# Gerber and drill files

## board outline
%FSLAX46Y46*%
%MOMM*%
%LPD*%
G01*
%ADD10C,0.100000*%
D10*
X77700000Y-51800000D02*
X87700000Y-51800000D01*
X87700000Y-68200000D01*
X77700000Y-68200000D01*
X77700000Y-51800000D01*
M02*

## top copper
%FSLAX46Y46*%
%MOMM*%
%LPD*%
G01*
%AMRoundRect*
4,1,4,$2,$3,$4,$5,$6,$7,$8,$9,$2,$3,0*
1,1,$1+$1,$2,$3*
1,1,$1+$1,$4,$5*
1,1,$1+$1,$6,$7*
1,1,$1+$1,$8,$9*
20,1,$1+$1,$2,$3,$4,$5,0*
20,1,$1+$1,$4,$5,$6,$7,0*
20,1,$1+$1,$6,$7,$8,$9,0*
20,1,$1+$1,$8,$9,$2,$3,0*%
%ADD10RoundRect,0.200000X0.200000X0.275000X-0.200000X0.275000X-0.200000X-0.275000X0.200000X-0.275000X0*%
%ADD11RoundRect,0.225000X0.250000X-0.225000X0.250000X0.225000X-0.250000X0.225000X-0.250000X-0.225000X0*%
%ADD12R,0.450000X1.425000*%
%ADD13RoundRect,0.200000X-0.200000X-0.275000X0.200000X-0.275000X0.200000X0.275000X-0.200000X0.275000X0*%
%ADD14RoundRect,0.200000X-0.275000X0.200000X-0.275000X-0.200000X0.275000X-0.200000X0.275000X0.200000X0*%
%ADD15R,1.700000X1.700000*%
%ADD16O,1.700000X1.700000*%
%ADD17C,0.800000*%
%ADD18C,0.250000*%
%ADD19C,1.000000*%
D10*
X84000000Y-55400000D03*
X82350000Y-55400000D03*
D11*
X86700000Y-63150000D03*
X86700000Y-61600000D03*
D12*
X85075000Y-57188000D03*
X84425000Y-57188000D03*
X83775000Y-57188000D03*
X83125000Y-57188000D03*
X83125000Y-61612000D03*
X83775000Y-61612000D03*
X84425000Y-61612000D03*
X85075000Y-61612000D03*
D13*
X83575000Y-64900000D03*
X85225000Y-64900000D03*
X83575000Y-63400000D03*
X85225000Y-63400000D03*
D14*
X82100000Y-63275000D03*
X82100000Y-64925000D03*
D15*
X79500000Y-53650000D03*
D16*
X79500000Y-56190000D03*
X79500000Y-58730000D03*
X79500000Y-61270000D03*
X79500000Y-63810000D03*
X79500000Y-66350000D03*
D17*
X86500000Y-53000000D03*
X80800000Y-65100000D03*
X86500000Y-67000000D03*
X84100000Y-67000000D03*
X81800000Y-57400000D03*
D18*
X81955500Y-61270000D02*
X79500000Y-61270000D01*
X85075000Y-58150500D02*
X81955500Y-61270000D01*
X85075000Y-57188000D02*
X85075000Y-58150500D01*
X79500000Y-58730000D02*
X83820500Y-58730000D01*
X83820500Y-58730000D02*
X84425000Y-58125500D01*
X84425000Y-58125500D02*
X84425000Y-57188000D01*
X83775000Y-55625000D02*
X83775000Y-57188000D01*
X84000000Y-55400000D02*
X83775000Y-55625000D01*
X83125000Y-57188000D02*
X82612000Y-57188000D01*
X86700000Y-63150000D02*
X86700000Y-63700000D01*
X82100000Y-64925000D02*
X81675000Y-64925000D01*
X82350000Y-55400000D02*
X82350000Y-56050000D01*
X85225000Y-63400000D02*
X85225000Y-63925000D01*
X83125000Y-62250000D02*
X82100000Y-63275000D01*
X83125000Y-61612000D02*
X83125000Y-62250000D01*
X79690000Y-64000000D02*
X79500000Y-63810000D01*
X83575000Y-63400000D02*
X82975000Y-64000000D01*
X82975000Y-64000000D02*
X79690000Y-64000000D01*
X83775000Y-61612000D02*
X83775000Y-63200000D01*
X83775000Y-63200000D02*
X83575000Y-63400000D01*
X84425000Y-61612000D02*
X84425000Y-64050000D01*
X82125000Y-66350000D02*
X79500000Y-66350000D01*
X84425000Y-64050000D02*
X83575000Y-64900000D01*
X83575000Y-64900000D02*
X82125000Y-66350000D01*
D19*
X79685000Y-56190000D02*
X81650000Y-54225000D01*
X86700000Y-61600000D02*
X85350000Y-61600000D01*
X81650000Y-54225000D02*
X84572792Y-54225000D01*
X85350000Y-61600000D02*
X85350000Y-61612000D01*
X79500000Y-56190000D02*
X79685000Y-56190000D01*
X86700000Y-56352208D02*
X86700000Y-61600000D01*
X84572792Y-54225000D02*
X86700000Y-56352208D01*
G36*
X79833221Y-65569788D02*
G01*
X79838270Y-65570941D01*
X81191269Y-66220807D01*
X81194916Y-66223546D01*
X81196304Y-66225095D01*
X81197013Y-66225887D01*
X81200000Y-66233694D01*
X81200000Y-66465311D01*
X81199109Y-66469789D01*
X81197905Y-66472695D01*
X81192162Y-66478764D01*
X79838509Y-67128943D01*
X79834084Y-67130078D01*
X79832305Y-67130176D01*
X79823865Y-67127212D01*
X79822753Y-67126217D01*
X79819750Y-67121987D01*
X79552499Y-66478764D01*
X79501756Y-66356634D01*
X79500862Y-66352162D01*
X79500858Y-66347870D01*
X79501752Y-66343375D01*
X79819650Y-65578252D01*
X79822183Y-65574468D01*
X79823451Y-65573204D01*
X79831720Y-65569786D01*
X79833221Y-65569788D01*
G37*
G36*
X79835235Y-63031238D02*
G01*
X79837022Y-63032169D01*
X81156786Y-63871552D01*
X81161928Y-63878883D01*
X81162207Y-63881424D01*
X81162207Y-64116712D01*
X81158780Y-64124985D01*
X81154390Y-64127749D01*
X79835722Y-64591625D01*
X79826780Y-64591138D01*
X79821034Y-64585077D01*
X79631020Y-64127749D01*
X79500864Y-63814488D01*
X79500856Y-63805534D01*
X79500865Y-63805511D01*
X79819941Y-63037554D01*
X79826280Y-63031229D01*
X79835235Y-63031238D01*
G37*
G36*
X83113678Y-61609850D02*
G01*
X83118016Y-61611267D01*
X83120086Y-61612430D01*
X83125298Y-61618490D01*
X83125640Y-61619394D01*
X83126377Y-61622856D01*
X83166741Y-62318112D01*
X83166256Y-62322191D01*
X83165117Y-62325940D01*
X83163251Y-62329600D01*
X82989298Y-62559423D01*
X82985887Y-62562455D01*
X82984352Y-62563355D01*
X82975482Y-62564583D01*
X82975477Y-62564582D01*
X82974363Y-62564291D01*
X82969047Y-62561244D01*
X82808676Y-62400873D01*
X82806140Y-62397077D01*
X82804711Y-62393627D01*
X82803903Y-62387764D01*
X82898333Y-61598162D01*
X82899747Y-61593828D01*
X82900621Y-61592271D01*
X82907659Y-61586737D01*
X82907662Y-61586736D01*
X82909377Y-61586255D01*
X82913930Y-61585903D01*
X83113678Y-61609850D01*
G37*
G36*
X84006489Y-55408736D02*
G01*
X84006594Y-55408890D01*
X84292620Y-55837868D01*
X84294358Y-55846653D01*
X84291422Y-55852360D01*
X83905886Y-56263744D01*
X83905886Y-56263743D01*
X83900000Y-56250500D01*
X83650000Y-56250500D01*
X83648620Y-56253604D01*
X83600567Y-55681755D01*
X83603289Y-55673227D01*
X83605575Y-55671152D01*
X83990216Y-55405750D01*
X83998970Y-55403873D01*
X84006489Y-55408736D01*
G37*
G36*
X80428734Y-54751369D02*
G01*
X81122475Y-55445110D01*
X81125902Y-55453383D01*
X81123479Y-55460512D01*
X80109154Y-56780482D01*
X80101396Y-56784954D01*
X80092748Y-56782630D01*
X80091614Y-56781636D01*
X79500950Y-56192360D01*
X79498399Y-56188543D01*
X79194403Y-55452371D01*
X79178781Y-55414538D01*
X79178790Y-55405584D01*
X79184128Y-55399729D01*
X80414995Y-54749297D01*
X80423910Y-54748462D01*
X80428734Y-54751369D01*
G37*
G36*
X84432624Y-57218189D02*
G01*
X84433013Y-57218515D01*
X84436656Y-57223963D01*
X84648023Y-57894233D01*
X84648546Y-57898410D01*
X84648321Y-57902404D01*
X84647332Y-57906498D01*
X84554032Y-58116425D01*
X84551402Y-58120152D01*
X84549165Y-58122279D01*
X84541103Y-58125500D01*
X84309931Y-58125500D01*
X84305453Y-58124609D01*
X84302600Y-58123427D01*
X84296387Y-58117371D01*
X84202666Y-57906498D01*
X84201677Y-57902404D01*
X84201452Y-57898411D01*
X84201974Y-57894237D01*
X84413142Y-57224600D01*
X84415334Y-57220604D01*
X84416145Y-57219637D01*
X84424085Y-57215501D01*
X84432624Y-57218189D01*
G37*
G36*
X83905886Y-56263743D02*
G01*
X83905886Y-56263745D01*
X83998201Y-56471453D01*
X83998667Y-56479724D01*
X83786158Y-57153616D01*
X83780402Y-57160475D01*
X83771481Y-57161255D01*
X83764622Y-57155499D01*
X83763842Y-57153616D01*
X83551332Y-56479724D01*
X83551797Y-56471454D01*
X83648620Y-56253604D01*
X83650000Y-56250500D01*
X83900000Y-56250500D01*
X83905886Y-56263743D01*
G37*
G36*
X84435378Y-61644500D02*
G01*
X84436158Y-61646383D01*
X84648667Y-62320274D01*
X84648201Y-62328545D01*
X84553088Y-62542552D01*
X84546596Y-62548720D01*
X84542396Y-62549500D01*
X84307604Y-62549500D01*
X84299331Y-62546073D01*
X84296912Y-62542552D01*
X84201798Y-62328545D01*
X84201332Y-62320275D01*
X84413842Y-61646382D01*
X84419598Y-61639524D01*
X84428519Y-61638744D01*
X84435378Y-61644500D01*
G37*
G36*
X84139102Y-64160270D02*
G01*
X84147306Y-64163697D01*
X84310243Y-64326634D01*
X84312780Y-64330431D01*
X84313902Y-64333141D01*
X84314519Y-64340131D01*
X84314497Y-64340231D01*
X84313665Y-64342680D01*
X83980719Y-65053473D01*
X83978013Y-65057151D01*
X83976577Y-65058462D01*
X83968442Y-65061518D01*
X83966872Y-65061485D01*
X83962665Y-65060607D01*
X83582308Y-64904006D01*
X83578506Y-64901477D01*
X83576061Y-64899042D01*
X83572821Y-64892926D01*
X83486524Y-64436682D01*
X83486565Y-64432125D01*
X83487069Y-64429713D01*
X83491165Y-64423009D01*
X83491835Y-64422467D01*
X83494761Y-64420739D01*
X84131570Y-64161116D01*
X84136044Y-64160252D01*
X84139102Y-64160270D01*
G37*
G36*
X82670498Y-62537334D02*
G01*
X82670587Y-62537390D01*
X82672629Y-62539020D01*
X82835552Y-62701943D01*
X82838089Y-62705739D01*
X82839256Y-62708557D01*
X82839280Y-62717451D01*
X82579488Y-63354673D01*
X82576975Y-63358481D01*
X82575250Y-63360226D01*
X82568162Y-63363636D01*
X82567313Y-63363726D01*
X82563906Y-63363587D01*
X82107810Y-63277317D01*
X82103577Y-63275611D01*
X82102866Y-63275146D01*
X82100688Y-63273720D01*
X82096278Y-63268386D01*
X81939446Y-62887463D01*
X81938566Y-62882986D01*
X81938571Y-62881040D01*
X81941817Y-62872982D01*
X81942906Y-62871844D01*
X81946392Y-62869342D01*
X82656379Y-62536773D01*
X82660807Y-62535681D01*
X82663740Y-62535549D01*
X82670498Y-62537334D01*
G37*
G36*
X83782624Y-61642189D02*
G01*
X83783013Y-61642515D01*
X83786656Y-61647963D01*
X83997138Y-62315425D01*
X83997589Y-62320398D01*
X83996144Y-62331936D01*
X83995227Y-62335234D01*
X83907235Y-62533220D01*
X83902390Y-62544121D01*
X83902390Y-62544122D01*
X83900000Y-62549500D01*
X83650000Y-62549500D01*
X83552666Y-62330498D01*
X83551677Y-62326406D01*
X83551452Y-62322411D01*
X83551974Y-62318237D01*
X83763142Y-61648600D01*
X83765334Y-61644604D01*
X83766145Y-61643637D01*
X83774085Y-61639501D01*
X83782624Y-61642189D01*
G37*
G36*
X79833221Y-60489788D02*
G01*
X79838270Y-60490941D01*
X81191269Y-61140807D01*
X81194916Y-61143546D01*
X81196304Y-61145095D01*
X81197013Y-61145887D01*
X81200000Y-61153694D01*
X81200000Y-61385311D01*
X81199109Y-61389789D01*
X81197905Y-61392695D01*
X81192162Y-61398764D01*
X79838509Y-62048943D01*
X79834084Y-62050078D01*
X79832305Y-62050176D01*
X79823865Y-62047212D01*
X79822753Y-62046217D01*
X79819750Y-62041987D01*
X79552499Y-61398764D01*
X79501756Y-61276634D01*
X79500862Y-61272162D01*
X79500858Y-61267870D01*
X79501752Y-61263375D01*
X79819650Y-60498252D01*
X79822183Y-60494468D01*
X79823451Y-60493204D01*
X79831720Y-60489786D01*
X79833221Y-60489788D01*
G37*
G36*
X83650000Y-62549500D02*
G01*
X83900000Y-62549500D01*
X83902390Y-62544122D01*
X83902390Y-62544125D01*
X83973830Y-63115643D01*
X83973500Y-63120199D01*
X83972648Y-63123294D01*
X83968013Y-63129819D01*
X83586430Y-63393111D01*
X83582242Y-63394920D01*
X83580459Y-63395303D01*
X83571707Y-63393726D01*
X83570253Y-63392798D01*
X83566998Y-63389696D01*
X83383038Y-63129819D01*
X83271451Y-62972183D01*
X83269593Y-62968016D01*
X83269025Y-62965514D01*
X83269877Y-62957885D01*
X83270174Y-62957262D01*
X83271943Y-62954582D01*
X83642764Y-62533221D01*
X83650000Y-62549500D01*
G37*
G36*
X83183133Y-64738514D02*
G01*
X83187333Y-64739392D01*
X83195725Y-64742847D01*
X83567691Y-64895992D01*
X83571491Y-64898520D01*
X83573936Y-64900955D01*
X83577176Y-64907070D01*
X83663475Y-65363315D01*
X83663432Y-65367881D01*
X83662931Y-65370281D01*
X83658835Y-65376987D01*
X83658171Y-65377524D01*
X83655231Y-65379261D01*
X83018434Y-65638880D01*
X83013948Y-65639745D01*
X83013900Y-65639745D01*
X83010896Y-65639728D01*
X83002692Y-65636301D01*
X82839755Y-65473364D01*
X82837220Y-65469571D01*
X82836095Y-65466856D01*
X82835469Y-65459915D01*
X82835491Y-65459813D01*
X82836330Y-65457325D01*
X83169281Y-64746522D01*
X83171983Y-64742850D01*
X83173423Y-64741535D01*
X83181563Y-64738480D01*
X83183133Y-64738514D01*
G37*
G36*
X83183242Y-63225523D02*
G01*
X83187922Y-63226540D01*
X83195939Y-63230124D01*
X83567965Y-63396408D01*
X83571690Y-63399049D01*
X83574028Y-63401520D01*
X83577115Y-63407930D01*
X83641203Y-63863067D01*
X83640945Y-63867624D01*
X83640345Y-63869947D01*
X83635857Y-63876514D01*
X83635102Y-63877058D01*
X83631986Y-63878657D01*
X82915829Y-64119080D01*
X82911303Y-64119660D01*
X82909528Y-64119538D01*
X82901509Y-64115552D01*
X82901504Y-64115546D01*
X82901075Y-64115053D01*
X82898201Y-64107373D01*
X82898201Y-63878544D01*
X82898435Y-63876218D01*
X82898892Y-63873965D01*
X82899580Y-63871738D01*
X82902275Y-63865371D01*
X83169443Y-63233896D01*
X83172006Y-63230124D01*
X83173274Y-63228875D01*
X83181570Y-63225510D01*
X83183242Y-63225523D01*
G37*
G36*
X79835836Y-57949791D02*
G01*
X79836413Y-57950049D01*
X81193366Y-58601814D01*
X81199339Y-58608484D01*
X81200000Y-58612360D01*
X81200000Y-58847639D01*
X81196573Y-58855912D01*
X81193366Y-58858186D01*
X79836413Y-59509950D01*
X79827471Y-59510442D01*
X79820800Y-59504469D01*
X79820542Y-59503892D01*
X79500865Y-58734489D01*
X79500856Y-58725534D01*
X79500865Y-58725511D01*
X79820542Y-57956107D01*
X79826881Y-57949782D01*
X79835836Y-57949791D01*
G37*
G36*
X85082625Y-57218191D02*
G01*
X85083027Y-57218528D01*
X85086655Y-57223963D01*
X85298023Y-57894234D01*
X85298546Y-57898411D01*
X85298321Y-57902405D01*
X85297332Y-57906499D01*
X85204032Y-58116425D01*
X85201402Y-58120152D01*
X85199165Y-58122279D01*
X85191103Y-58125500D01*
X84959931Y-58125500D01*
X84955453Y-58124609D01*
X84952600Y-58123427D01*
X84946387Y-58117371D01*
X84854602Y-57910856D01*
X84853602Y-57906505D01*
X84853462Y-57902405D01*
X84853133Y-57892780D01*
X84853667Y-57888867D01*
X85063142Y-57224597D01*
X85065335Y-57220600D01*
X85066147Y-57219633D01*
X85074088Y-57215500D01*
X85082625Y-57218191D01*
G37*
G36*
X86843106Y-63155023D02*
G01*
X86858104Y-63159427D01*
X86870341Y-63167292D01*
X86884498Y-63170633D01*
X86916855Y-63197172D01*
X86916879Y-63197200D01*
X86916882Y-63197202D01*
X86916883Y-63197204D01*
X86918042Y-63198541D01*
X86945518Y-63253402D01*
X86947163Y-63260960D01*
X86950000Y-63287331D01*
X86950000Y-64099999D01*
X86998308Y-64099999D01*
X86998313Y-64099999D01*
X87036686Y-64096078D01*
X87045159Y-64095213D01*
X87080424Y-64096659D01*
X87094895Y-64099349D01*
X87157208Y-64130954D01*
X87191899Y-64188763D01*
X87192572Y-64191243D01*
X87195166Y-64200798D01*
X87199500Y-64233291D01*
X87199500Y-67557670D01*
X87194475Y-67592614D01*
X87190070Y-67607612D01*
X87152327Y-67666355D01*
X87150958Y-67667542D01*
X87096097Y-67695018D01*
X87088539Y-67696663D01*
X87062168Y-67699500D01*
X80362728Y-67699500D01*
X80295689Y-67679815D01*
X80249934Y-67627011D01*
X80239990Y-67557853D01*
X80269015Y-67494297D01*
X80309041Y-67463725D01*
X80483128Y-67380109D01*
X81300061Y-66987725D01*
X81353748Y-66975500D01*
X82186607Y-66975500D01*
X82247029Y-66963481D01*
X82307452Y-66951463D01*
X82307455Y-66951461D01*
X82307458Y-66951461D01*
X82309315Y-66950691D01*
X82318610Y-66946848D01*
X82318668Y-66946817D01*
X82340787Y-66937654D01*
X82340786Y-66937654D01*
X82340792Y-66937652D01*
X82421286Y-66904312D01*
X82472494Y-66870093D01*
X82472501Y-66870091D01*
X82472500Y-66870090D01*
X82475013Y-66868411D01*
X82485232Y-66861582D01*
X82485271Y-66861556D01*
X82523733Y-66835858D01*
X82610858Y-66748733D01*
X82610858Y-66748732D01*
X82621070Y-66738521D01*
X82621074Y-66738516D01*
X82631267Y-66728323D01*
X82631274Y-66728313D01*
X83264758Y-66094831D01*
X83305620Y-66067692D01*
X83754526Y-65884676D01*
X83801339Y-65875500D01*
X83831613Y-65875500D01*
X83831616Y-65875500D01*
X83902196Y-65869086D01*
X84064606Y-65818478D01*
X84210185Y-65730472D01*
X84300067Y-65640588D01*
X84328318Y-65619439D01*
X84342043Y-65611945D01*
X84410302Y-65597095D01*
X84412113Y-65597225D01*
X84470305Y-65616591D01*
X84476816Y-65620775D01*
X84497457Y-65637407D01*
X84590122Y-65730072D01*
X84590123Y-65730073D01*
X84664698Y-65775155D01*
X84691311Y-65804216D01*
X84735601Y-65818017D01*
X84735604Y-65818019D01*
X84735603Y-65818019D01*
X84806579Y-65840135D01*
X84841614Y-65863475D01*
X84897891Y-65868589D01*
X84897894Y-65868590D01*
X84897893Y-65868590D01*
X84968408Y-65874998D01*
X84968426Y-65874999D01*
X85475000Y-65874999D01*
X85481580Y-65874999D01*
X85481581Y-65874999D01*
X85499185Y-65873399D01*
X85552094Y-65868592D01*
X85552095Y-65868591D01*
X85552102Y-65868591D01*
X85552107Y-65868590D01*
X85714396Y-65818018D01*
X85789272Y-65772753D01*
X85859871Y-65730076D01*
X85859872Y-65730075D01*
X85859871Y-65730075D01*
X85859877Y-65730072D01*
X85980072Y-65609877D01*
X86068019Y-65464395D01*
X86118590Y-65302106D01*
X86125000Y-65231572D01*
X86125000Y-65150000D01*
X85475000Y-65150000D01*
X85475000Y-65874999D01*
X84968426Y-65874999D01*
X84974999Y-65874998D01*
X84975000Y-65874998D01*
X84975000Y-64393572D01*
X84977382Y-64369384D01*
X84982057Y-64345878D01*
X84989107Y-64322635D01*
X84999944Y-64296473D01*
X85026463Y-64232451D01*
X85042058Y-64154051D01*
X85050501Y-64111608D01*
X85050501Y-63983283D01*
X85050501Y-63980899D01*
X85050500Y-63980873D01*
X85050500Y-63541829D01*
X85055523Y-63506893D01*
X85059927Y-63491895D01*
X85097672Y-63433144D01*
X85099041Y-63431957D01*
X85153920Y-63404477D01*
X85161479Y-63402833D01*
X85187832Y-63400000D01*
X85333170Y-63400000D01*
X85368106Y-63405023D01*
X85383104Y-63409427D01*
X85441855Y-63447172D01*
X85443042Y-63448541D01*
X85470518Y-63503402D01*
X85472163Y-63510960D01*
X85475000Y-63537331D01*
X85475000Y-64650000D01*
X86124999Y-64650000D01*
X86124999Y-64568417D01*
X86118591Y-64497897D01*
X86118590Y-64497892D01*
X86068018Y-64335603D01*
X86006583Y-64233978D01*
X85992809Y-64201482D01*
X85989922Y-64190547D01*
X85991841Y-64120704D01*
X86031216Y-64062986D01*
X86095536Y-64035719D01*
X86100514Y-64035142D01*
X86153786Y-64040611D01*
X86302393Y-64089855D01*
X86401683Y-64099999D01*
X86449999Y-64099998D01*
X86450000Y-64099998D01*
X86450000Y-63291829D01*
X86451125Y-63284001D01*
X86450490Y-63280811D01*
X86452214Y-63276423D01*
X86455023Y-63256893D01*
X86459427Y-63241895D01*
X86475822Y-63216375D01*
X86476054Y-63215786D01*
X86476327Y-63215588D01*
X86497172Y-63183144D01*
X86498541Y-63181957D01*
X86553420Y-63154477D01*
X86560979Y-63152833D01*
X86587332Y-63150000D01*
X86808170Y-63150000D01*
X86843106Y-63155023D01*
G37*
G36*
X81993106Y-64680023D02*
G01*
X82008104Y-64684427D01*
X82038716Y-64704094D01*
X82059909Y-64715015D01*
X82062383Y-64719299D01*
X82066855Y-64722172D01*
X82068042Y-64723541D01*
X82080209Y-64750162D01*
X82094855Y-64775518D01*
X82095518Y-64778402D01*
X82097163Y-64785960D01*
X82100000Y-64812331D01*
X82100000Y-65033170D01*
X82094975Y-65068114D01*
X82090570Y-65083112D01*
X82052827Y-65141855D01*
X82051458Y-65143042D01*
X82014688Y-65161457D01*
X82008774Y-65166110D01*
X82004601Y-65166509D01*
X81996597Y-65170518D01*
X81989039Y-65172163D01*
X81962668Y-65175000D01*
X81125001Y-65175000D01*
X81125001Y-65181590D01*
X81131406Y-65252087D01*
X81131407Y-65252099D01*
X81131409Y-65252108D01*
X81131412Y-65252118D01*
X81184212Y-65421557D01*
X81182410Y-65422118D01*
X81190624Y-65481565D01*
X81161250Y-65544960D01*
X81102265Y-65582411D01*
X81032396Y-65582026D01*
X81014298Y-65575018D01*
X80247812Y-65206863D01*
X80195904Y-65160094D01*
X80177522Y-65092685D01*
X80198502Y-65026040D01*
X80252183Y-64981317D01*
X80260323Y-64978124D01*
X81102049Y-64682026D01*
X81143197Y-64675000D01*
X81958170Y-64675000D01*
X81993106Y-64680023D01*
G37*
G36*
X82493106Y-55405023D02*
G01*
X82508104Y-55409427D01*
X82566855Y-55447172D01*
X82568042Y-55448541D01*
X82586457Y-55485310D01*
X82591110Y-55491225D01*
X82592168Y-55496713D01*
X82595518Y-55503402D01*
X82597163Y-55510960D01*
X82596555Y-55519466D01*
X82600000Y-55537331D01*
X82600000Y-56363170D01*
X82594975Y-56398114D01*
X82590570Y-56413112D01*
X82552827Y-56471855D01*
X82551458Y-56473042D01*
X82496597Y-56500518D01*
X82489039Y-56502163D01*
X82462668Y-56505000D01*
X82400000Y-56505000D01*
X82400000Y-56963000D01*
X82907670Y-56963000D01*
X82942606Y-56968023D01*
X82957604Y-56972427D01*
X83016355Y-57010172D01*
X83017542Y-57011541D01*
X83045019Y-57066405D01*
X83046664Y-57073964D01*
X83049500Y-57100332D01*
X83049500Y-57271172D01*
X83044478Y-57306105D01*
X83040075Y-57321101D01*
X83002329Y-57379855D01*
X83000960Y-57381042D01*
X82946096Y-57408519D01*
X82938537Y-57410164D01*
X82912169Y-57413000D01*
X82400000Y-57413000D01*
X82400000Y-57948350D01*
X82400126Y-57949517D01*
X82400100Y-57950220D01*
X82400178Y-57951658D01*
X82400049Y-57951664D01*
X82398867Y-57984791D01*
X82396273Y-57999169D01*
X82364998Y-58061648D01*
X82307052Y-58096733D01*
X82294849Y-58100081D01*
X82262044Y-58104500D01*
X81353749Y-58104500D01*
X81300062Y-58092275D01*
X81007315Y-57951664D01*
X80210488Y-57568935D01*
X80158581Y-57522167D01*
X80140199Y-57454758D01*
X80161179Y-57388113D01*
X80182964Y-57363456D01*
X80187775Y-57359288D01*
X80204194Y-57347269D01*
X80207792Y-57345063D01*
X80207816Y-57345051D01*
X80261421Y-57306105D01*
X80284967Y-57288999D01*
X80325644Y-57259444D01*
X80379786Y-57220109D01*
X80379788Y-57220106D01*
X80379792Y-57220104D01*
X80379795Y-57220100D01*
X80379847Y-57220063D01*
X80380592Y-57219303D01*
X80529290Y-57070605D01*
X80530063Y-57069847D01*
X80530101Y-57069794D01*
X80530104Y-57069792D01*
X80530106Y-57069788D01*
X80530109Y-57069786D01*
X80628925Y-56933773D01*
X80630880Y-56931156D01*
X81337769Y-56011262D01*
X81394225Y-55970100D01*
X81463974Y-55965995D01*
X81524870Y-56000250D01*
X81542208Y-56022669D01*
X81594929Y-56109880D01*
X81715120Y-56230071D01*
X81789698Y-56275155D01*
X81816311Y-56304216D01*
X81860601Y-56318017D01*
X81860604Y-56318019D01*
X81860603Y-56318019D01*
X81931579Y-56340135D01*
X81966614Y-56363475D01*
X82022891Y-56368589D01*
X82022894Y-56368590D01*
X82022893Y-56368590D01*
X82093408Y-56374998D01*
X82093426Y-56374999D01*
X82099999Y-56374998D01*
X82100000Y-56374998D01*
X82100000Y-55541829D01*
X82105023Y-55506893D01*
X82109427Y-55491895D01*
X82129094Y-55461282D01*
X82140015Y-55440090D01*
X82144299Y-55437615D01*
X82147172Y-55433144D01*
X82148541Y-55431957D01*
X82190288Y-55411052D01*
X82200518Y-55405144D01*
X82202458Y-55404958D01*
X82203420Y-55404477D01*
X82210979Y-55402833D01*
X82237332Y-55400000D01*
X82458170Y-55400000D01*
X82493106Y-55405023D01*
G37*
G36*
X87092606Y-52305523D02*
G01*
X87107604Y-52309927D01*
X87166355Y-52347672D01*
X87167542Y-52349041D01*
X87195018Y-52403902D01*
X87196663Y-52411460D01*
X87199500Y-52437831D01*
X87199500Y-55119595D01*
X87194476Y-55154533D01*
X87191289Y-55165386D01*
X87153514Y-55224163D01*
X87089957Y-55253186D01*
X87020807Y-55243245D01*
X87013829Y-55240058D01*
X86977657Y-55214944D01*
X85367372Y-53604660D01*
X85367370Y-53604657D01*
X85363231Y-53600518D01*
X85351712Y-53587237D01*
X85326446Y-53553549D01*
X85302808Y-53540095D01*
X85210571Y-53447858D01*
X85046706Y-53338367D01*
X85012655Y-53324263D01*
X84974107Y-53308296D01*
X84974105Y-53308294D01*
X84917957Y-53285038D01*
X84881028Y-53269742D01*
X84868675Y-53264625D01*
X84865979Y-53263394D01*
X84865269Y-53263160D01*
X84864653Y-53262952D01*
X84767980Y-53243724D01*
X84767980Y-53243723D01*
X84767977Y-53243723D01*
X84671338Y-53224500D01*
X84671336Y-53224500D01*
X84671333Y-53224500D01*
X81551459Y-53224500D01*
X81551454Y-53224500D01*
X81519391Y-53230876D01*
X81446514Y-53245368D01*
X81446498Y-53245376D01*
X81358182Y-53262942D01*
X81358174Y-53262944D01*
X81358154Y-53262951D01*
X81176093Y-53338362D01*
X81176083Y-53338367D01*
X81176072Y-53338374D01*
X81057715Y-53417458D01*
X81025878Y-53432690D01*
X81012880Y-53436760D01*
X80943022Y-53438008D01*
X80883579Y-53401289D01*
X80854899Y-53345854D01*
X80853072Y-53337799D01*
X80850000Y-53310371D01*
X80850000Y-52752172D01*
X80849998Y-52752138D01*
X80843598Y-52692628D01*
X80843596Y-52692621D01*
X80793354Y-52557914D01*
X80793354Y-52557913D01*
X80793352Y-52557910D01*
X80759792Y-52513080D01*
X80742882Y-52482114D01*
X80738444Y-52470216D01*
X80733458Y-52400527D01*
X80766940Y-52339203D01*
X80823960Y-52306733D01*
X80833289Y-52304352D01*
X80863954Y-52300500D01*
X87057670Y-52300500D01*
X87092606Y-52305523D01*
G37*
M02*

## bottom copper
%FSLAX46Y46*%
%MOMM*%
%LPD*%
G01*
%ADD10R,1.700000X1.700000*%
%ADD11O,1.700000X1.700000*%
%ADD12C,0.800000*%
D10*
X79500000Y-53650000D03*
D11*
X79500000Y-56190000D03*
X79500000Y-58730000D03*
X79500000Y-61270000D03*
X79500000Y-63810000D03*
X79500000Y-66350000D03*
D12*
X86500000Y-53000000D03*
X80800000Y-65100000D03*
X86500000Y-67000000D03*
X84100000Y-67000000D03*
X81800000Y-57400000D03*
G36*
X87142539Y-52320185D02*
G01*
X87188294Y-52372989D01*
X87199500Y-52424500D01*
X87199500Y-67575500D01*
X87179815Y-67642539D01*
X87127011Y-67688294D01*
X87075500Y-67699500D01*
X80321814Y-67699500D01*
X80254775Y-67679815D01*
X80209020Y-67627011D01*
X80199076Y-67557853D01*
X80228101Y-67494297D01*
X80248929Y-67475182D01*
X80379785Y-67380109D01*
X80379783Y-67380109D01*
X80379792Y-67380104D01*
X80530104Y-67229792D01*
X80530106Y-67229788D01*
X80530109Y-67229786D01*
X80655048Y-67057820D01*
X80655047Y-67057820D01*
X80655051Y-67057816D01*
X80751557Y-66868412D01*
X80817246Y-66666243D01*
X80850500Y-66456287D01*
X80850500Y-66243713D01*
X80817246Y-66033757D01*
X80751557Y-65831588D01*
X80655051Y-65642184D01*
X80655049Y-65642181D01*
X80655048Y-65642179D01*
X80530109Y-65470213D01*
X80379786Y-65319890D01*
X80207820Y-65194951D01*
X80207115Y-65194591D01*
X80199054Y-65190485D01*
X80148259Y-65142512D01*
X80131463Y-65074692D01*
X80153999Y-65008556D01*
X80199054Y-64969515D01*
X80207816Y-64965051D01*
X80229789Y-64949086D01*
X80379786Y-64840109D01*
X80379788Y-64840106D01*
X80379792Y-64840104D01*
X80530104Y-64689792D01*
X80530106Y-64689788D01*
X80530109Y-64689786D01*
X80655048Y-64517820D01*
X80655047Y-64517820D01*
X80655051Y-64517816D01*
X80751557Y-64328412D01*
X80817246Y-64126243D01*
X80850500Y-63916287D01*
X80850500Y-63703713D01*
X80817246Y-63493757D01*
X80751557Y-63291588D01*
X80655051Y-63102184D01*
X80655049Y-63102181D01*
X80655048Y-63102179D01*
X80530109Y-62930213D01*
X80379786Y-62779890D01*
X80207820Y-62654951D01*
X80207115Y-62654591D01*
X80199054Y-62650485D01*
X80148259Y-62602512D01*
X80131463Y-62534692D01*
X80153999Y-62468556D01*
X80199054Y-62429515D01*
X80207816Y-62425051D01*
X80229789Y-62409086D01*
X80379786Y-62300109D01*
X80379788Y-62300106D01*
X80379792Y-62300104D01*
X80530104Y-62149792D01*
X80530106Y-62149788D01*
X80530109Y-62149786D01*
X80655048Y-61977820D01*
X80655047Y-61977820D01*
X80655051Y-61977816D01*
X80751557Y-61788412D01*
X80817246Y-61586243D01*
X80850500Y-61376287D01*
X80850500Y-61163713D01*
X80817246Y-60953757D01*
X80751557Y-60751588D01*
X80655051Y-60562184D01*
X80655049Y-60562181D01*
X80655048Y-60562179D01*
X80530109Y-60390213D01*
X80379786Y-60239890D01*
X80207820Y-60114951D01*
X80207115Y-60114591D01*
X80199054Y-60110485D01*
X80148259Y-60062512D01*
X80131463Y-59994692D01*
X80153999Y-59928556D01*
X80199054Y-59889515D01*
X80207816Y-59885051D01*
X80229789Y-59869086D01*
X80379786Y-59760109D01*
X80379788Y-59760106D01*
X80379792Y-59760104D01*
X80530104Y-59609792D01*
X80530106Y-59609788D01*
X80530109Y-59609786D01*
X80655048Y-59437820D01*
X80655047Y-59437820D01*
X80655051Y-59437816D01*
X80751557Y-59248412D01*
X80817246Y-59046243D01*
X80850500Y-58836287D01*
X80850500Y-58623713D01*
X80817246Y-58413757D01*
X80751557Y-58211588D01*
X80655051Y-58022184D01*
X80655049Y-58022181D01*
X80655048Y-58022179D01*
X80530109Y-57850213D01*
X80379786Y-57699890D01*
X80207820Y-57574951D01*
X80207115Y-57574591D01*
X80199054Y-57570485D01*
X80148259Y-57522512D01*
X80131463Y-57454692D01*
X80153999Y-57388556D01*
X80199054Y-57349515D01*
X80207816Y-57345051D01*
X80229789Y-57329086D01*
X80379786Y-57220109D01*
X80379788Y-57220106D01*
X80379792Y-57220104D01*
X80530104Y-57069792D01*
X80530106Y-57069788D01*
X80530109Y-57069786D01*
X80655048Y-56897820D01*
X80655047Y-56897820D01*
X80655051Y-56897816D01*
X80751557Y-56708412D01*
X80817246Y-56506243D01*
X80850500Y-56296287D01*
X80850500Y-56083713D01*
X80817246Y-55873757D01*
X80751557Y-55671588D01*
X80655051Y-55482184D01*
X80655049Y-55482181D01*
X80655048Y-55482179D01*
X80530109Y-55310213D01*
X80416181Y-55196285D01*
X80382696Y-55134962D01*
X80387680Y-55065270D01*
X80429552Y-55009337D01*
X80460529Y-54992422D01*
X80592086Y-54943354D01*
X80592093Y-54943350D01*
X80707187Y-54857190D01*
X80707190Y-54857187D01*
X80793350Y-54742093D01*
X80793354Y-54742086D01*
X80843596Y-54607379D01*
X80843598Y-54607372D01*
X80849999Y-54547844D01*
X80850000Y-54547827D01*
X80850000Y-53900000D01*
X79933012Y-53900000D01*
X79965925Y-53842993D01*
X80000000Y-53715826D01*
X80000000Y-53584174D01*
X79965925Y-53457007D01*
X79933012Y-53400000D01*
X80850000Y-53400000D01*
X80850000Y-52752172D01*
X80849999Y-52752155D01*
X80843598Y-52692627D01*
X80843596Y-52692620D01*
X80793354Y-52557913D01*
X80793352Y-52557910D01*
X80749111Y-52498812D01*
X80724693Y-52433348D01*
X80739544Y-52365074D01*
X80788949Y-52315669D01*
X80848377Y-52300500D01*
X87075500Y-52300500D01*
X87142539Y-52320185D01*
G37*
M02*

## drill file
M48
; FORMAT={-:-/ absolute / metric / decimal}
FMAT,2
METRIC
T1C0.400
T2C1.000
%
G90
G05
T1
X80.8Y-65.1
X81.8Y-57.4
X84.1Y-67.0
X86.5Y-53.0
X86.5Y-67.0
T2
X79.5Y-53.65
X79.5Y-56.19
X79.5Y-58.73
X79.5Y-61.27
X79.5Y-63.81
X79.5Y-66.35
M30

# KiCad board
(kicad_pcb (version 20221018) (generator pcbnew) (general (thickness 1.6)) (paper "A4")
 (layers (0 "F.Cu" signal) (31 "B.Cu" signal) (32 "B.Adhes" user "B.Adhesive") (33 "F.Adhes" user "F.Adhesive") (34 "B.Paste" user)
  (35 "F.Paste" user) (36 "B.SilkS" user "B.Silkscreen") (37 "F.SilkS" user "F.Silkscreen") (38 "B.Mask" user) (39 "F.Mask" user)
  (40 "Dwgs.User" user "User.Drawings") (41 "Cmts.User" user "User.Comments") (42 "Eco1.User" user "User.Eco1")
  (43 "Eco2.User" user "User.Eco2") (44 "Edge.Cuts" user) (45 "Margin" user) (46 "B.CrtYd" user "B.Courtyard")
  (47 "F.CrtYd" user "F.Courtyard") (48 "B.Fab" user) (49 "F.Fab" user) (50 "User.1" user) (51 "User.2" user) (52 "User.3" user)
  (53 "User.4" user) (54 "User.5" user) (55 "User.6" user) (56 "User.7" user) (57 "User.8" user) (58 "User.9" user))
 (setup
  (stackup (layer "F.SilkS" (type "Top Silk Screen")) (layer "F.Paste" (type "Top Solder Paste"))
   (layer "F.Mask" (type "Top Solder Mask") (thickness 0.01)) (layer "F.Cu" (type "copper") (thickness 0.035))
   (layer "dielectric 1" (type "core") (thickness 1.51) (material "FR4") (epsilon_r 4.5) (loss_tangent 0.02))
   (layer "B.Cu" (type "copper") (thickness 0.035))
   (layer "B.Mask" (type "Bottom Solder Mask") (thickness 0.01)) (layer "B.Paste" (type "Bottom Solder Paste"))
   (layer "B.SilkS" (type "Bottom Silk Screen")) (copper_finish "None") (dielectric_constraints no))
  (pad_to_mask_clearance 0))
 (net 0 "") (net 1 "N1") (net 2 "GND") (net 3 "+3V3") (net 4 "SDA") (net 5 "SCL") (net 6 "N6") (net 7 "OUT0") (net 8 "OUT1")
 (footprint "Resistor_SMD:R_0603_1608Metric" (layer "F.Cu") (at 83.175 55.4 180)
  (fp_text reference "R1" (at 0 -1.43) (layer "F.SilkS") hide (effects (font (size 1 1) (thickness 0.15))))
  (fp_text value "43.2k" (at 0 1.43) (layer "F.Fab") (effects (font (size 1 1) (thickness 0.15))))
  (pad "1" smd roundrect (at -0.825 0 180) (size 0.8 0.95) (layers "F.Cu" "F.Paste" "F.Mask") (roundrect_rratio 0.25) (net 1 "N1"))
  (pad "2" smd roundrect (at 0.825 0 180) (size 0.8 0.95) (layers "F.Cu" "F.Paste" "F.Mask") (roundrect_rratio 0.25) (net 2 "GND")))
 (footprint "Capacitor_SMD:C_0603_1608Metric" (layer "F.Cu") (at 86.7 62.375 90)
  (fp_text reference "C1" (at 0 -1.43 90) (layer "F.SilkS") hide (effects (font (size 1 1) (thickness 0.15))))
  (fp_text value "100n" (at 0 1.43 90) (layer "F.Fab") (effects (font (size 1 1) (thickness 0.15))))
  (pad "1" smd roundrect (at -0.775 0 90) (size 0.9 0.95) (layers "F.Cu" "F.Paste" "F.Mask") (roundrect_rratio 0.25) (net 2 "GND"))
  (pad "2" smd roundrect (at 0.775 0 90) (size 0.9 0.95) (layers "F.Cu" "F.Paste" "F.Mask") (roundrect_rratio 0.25) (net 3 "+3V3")))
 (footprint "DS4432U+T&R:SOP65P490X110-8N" (layer "F.Cu") (at 84.1 59.4 -90)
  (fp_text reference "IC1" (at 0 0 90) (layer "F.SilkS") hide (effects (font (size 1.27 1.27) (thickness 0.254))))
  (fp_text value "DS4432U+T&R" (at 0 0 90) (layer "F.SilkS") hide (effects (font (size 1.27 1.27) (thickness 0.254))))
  (pad "1" smd rect (at -2.212 -0.975) (size 0.45 1.425) (layers "F.Cu" "F.Paste" "F.Mask") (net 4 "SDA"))
  (pad "2" smd rect (at -2.212 -0.325) (size 0.45 1.425) (layers "F.Cu" "F.Paste" "F.Mask") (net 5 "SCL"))
  (pad "3" smd rect (at -2.212 0.325) (size 0.45 1.425) (layers "F.Cu" "F.Paste" "F.Mask") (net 1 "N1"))
  (pad "4" smd rect (at -2.212 0.975) (size 0.45 1.425) (layers "F.Cu" "F.Paste" "F.Mask") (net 2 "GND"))
  (pad "5" smd rect (at 2.212 0.975) (size 0.45 1.425) (layers "F.Cu" "F.Paste" "F.Mask") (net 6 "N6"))
  (pad "6" smd rect (at 2.212 0.325) (size 0.45 1.425) (layers "F.Cu" "F.Paste" "F.Mask") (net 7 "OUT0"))
  (pad "7" smd rect (at 2.212 -0.325) (size 0.45 1.425) (layers "F.Cu" "F.Paste" "F.Mask") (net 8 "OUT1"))
  (pad "8" smd rect (at 2.212 -0.975) (size 0.45 1.425) (layers "F.Cu" "F.Paste" "F.Mask") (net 3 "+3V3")))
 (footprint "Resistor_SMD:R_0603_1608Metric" (layer "F.Cu") (at 84.4 64.9)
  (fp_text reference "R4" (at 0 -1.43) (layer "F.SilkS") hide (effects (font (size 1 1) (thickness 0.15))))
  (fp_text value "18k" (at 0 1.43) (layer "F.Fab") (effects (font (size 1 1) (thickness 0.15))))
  (pad "1" smd roundrect (at -0.825 0) (size 0.8 0.95) (layers "F.Cu" "F.Paste" "F.Mask") (roundrect_rratio 0.25) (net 8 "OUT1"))
  (pad "2" smd roundrect (at 0.825 0) (size 0.8 0.95) (layers "F.Cu" "F.Paste" "F.Mask") (roundrect_rratio 0.25) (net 2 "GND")))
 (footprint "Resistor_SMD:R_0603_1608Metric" (layer "F.Cu") (at 84.4 63.4)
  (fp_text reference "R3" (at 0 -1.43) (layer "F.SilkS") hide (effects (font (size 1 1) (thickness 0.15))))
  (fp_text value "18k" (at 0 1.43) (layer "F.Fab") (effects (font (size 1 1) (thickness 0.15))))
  (pad "1" smd roundrect (at -0.825 0) (size 0.8 0.95) (layers "F.Cu" "F.Paste" "F.Mask") (roundrect_rratio 0.25) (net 7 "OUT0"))
  (pad "2" smd roundrect (at 0.825 0) (size 0.8 0.95) (layers "F.Cu" "F.Paste" "F.Mask") (roundrect_rratio 0.25) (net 2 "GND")))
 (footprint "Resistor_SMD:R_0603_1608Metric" (layer "F.Cu") (at 82.1 64.1 -90)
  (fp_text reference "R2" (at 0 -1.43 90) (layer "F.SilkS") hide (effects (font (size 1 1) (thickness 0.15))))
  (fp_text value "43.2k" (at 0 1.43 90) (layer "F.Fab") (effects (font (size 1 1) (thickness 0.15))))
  (pad "1" smd roundrect (at -0.825 0 270) (size 0.8 0.95) (layers "F.Cu" "F.Paste" "F.Mask") (roundrect_rratio 0.25) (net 6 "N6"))
  (pad "2" smd roundrect (at 0.825 0 270) (size 0.8 0.95) (layers "F.Cu" "F.Paste" "F.Mask") (roundrect_rratio 0.25) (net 2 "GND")))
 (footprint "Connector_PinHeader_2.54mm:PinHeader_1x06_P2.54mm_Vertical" (layer "B.Cu") (at 79.5 53.65 180)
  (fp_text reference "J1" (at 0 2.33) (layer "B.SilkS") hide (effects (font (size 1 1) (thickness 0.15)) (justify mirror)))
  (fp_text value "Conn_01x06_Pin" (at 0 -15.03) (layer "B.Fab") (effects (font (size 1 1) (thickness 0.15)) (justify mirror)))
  (pad "1" thru_hole rect (at 0 0 180) (size 1.7 1.7) (drill 1) (layers "*.Cu" "*.Mask") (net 2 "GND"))
  (pad "2" thru_hole oval (at 0 -2.54 180) (size 1.7 1.7) (drill 1) (layers "*.Cu" "*.Mask") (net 3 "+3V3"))
  (pad "3" thru_hole oval (at 0 -5.08 180) (size 1.7 1.7) (drill 1) (layers "*.Cu" "*.Mask") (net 5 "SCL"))
  (pad "4" thru_hole oval (at 0 -7.62 180) (size 1.7 1.7) (drill 1) (layers "*.Cu" "*.Mask") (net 4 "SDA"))
  (pad "5" thru_hole oval (at 0 -10.16 180) (size 1.7 1.7) (drill 1) (layers "*.Cu" "*.Mask") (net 7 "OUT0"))
  (pad "6" thru_hole oval (at 0 -12.7 180) (size 1.7 1.7) (drill 1) (layers "*.Cu" "*.Mask") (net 8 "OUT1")))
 (gr_rect (start 77.7 51.8) (end 87.7 68.2) (stroke (width 0.1) (type default)) (fill none) (layer "Edge.Cuts"))
 (segment (start 81.9555 61.27) (end 79.5 61.27) (width 0.25) (layer "F.Cu") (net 4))
 (segment (start 85.075 58.1505) (end 81.9555 61.27) (width 0.25) (layer "F.Cu") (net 4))
 (segment (start 85.075 57.188) (end 85.075 58.1505) (width 0.25) (layer "F.Cu") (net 4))
 (segment (start 79.5 58.73) (end 83.8205 58.73) (width 0.25) (layer "F.Cu") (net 5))
 (segment (start 83.8205 58.73) (end 84.425 58.1255) (width 0.25) (layer "F.Cu") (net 5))
 (segment (start 84.425 58.1255) (end 84.425 57.188) (width 0.25) (layer "F.Cu") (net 5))
 (segment (start 83.775 55.625) (end 83.775 57.188) (width 0.25) (layer "F.Cu") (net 1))
 (segment (start 84 55.4) (end 83.775 55.625) (width 0.25) (layer "F.Cu") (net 1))
 (segment (start 83.125 57.188) (end 82.612 57.188) (width 0.25) (layer "F.Cu") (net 2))
 (segment (start 86.7 63.15) (end 86.7 63.7) (width 0.25) (layer "F.Cu") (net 2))
 (segment (start 82.1 64.925) (end 81.675 64.925) (width 0.25) (layer "F.Cu") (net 2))
 (segment (start 82.35 55.4) (end 82.35 56.05) (width 0.25) (layer "F.Cu") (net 2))
 (segment (start 85.225 63.4) (end 85.225 63.925) (width 0.25) (layer "F.Cu") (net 2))
 (via (at 86.5 53) (size 0.8) (drill 0.4) (layers "F.Cu" "B.Cu") (free) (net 2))
 (via (at 80.8 65.1) (size 0.8) (drill 0.4) (layers "F.Cu" "B.Cu") (free) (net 2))
 (via (at 86.5 67) (size 0.8) (drill 0.4) (layers "F.Cu" "B.Cu") (free) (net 2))
 (via (at 84.1 67) (size 0.8) (drill 0.4) (layers "F.Cu" "B.Cu") (free) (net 2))
 (via (at 81.8 57.4) (size 0.8) (drill 0.4) (layers "F.Cu" "B.Cu") (free) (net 2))
 (segment (start 83.125 62.25) (end 82.1 63.275) (width 0.25) (layer "F.Cu") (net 6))
 (segment (start 83.125 61.612) (end 83.125 62.25) (width 0.25) (layer "F.Cu") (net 6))
 (segment (start 79.69 64) (end 79.5 63.81) (width 0.25) (layer "F.Cu") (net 7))
 (segment (start 83.575 63.4) (end 82.975 64) (width 0.25) (layer "F.Cu") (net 7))
 (segment (start 82.975 64) (end 79.69 64) (width 0.25) (layer "F.Cu") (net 7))
 (segment (start 83.775 61.612) (end 83.775 63.2) (width 0.25) (layer "F.Cu") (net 7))
 (segment (start 83.775 63.2) (end 83.575 63.4) (width 0.25) (layer "F.Cu") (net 7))
 (segment (start 84.425 61.612) (end 84.425 64.05) (width 0.25) (layer "F.Cu") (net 8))
 (segment (start 82.125 66.35) (end 79.5 66.35) (width 0.25) (layer "F.Cu") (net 8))
 (segment (start 84.425 64.05) (end 83.575 64.9) (width 0.25) (layer "F.Cu") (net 8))
 (segment (start 83.575 64.9) (end 82.125 66.35) (width 0.25) (layer "F.Cu") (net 8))
 (segment (start 79.685 56.19) (end 81.65 54.225) (width 1) (layer "F.Cu") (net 3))
 (segment (start 86.7 61.6) (end 85.35 61.6) (width 1) (layer "F.Cu") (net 3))
 (segment (start 81.65 54.225) (end 84.572792 54.225) (width 1) (layer "F.Cu") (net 3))
 (segment (start 85.35 61.6) (end 85.35 61.612) (width 1) (layer "F.Cu") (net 3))
 (segment (start 79.5 56.19) (end 79.685 56.19) (width 1) (layer "F.Cu") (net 3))
 (segment (start 86.7 56.352208) (end 86.7 61.6) (width 1) (layer "F.Cu") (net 3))
 (segment (start 84.572792 54.225) (end 86.7 56.352208) (width 1) (layer "F.Cu") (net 3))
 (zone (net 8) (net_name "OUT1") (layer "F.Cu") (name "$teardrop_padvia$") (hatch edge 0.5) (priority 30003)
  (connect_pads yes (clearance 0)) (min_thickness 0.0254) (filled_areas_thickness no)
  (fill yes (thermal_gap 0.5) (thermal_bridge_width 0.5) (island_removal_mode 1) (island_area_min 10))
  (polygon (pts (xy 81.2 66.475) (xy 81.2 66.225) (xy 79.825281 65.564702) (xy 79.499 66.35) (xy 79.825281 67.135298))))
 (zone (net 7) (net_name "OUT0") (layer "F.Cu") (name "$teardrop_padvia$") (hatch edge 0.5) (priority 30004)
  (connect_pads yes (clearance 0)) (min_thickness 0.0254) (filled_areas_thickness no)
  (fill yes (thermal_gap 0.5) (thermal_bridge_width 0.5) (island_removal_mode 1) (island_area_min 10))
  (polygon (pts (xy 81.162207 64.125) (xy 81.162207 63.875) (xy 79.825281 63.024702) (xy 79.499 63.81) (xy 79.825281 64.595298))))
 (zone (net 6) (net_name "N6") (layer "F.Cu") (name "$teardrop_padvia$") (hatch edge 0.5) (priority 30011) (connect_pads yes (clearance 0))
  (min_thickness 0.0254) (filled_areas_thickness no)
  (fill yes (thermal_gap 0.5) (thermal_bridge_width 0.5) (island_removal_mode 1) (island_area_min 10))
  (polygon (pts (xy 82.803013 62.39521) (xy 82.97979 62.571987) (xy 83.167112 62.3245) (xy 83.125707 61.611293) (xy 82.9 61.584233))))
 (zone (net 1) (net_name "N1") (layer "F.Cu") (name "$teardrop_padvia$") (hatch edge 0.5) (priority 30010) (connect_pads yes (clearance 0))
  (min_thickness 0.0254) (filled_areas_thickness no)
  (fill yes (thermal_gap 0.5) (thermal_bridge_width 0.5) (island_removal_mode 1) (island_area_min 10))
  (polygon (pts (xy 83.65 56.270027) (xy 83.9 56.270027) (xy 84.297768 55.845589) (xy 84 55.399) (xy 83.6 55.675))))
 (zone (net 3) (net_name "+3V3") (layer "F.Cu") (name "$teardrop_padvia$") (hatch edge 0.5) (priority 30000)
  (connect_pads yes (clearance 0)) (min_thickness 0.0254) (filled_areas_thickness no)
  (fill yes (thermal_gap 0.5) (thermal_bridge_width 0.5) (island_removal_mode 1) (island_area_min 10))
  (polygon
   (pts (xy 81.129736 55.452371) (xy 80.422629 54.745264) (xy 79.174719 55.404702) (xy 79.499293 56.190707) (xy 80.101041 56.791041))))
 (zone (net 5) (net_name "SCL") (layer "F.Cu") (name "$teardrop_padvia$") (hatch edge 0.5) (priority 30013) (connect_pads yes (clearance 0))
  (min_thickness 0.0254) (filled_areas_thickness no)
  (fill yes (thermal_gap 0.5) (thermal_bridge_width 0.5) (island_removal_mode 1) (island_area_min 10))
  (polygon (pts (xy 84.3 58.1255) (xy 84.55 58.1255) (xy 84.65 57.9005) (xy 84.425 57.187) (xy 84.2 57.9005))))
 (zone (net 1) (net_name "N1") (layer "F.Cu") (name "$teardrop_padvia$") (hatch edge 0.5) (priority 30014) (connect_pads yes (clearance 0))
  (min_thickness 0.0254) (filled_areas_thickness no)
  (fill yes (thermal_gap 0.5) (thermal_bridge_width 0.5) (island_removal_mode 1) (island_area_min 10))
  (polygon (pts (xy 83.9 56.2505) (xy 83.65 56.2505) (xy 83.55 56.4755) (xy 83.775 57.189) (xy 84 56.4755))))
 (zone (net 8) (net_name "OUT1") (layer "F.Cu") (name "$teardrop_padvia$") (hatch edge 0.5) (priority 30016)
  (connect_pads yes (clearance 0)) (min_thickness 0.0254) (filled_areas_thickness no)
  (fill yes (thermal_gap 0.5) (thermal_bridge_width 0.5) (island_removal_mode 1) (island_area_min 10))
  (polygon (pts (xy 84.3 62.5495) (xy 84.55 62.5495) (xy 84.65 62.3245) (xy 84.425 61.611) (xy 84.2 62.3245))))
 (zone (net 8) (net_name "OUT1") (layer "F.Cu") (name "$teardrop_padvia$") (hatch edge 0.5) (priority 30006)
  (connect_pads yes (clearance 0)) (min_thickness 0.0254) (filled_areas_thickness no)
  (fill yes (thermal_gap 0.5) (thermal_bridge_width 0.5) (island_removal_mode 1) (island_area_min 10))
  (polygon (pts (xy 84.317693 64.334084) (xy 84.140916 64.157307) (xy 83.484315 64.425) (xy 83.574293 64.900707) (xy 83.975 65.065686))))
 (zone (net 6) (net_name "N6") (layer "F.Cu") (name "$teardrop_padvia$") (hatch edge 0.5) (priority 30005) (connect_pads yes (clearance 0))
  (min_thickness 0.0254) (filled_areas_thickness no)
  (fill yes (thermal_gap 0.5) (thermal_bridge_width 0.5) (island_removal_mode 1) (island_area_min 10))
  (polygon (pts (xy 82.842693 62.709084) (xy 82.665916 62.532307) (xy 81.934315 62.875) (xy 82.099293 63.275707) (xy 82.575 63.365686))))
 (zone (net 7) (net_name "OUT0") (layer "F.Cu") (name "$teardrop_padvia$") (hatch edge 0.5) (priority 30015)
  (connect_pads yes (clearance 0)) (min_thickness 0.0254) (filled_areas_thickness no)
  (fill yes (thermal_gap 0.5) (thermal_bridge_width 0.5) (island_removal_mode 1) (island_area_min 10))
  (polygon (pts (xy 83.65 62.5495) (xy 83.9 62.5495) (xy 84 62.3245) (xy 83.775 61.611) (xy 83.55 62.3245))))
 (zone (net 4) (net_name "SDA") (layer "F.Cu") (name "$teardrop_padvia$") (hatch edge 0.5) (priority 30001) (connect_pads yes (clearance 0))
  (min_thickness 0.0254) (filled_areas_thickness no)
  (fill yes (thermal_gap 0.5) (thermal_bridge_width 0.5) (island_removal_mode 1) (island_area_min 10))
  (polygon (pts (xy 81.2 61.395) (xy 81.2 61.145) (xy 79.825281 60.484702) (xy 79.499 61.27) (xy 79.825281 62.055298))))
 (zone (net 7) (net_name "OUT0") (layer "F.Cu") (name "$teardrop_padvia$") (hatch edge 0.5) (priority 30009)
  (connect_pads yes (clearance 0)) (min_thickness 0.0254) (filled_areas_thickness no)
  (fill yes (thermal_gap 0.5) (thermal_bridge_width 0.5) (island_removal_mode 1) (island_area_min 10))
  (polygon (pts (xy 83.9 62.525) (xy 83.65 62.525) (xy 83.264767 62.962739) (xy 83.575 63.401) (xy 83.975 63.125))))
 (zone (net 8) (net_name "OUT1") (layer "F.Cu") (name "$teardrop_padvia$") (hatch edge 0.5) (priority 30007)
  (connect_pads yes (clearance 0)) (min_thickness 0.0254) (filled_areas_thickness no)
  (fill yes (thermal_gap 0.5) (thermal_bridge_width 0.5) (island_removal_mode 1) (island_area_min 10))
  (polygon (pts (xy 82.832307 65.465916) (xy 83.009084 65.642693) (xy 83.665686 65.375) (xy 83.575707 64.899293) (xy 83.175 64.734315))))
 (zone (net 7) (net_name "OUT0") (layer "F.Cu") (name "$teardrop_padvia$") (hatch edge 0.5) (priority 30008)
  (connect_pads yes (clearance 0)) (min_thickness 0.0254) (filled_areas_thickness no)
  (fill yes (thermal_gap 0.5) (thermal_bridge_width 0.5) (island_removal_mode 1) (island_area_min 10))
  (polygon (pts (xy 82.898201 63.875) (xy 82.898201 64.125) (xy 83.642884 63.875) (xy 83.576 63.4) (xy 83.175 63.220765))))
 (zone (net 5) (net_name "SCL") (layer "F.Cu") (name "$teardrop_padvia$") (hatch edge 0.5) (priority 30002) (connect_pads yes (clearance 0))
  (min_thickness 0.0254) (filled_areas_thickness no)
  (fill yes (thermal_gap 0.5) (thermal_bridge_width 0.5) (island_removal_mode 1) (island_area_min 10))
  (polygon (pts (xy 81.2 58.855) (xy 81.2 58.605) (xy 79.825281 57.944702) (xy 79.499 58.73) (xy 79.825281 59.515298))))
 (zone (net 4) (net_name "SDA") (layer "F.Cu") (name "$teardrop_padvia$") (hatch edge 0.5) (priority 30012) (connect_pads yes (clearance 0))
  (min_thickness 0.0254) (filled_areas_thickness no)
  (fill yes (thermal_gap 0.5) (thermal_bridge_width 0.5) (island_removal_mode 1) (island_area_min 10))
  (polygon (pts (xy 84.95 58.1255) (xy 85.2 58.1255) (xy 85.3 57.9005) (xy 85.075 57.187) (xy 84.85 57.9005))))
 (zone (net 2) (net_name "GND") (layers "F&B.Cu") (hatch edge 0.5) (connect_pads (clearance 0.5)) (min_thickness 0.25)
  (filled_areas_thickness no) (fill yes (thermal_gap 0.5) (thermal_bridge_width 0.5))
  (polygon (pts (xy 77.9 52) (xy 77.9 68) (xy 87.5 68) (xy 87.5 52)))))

